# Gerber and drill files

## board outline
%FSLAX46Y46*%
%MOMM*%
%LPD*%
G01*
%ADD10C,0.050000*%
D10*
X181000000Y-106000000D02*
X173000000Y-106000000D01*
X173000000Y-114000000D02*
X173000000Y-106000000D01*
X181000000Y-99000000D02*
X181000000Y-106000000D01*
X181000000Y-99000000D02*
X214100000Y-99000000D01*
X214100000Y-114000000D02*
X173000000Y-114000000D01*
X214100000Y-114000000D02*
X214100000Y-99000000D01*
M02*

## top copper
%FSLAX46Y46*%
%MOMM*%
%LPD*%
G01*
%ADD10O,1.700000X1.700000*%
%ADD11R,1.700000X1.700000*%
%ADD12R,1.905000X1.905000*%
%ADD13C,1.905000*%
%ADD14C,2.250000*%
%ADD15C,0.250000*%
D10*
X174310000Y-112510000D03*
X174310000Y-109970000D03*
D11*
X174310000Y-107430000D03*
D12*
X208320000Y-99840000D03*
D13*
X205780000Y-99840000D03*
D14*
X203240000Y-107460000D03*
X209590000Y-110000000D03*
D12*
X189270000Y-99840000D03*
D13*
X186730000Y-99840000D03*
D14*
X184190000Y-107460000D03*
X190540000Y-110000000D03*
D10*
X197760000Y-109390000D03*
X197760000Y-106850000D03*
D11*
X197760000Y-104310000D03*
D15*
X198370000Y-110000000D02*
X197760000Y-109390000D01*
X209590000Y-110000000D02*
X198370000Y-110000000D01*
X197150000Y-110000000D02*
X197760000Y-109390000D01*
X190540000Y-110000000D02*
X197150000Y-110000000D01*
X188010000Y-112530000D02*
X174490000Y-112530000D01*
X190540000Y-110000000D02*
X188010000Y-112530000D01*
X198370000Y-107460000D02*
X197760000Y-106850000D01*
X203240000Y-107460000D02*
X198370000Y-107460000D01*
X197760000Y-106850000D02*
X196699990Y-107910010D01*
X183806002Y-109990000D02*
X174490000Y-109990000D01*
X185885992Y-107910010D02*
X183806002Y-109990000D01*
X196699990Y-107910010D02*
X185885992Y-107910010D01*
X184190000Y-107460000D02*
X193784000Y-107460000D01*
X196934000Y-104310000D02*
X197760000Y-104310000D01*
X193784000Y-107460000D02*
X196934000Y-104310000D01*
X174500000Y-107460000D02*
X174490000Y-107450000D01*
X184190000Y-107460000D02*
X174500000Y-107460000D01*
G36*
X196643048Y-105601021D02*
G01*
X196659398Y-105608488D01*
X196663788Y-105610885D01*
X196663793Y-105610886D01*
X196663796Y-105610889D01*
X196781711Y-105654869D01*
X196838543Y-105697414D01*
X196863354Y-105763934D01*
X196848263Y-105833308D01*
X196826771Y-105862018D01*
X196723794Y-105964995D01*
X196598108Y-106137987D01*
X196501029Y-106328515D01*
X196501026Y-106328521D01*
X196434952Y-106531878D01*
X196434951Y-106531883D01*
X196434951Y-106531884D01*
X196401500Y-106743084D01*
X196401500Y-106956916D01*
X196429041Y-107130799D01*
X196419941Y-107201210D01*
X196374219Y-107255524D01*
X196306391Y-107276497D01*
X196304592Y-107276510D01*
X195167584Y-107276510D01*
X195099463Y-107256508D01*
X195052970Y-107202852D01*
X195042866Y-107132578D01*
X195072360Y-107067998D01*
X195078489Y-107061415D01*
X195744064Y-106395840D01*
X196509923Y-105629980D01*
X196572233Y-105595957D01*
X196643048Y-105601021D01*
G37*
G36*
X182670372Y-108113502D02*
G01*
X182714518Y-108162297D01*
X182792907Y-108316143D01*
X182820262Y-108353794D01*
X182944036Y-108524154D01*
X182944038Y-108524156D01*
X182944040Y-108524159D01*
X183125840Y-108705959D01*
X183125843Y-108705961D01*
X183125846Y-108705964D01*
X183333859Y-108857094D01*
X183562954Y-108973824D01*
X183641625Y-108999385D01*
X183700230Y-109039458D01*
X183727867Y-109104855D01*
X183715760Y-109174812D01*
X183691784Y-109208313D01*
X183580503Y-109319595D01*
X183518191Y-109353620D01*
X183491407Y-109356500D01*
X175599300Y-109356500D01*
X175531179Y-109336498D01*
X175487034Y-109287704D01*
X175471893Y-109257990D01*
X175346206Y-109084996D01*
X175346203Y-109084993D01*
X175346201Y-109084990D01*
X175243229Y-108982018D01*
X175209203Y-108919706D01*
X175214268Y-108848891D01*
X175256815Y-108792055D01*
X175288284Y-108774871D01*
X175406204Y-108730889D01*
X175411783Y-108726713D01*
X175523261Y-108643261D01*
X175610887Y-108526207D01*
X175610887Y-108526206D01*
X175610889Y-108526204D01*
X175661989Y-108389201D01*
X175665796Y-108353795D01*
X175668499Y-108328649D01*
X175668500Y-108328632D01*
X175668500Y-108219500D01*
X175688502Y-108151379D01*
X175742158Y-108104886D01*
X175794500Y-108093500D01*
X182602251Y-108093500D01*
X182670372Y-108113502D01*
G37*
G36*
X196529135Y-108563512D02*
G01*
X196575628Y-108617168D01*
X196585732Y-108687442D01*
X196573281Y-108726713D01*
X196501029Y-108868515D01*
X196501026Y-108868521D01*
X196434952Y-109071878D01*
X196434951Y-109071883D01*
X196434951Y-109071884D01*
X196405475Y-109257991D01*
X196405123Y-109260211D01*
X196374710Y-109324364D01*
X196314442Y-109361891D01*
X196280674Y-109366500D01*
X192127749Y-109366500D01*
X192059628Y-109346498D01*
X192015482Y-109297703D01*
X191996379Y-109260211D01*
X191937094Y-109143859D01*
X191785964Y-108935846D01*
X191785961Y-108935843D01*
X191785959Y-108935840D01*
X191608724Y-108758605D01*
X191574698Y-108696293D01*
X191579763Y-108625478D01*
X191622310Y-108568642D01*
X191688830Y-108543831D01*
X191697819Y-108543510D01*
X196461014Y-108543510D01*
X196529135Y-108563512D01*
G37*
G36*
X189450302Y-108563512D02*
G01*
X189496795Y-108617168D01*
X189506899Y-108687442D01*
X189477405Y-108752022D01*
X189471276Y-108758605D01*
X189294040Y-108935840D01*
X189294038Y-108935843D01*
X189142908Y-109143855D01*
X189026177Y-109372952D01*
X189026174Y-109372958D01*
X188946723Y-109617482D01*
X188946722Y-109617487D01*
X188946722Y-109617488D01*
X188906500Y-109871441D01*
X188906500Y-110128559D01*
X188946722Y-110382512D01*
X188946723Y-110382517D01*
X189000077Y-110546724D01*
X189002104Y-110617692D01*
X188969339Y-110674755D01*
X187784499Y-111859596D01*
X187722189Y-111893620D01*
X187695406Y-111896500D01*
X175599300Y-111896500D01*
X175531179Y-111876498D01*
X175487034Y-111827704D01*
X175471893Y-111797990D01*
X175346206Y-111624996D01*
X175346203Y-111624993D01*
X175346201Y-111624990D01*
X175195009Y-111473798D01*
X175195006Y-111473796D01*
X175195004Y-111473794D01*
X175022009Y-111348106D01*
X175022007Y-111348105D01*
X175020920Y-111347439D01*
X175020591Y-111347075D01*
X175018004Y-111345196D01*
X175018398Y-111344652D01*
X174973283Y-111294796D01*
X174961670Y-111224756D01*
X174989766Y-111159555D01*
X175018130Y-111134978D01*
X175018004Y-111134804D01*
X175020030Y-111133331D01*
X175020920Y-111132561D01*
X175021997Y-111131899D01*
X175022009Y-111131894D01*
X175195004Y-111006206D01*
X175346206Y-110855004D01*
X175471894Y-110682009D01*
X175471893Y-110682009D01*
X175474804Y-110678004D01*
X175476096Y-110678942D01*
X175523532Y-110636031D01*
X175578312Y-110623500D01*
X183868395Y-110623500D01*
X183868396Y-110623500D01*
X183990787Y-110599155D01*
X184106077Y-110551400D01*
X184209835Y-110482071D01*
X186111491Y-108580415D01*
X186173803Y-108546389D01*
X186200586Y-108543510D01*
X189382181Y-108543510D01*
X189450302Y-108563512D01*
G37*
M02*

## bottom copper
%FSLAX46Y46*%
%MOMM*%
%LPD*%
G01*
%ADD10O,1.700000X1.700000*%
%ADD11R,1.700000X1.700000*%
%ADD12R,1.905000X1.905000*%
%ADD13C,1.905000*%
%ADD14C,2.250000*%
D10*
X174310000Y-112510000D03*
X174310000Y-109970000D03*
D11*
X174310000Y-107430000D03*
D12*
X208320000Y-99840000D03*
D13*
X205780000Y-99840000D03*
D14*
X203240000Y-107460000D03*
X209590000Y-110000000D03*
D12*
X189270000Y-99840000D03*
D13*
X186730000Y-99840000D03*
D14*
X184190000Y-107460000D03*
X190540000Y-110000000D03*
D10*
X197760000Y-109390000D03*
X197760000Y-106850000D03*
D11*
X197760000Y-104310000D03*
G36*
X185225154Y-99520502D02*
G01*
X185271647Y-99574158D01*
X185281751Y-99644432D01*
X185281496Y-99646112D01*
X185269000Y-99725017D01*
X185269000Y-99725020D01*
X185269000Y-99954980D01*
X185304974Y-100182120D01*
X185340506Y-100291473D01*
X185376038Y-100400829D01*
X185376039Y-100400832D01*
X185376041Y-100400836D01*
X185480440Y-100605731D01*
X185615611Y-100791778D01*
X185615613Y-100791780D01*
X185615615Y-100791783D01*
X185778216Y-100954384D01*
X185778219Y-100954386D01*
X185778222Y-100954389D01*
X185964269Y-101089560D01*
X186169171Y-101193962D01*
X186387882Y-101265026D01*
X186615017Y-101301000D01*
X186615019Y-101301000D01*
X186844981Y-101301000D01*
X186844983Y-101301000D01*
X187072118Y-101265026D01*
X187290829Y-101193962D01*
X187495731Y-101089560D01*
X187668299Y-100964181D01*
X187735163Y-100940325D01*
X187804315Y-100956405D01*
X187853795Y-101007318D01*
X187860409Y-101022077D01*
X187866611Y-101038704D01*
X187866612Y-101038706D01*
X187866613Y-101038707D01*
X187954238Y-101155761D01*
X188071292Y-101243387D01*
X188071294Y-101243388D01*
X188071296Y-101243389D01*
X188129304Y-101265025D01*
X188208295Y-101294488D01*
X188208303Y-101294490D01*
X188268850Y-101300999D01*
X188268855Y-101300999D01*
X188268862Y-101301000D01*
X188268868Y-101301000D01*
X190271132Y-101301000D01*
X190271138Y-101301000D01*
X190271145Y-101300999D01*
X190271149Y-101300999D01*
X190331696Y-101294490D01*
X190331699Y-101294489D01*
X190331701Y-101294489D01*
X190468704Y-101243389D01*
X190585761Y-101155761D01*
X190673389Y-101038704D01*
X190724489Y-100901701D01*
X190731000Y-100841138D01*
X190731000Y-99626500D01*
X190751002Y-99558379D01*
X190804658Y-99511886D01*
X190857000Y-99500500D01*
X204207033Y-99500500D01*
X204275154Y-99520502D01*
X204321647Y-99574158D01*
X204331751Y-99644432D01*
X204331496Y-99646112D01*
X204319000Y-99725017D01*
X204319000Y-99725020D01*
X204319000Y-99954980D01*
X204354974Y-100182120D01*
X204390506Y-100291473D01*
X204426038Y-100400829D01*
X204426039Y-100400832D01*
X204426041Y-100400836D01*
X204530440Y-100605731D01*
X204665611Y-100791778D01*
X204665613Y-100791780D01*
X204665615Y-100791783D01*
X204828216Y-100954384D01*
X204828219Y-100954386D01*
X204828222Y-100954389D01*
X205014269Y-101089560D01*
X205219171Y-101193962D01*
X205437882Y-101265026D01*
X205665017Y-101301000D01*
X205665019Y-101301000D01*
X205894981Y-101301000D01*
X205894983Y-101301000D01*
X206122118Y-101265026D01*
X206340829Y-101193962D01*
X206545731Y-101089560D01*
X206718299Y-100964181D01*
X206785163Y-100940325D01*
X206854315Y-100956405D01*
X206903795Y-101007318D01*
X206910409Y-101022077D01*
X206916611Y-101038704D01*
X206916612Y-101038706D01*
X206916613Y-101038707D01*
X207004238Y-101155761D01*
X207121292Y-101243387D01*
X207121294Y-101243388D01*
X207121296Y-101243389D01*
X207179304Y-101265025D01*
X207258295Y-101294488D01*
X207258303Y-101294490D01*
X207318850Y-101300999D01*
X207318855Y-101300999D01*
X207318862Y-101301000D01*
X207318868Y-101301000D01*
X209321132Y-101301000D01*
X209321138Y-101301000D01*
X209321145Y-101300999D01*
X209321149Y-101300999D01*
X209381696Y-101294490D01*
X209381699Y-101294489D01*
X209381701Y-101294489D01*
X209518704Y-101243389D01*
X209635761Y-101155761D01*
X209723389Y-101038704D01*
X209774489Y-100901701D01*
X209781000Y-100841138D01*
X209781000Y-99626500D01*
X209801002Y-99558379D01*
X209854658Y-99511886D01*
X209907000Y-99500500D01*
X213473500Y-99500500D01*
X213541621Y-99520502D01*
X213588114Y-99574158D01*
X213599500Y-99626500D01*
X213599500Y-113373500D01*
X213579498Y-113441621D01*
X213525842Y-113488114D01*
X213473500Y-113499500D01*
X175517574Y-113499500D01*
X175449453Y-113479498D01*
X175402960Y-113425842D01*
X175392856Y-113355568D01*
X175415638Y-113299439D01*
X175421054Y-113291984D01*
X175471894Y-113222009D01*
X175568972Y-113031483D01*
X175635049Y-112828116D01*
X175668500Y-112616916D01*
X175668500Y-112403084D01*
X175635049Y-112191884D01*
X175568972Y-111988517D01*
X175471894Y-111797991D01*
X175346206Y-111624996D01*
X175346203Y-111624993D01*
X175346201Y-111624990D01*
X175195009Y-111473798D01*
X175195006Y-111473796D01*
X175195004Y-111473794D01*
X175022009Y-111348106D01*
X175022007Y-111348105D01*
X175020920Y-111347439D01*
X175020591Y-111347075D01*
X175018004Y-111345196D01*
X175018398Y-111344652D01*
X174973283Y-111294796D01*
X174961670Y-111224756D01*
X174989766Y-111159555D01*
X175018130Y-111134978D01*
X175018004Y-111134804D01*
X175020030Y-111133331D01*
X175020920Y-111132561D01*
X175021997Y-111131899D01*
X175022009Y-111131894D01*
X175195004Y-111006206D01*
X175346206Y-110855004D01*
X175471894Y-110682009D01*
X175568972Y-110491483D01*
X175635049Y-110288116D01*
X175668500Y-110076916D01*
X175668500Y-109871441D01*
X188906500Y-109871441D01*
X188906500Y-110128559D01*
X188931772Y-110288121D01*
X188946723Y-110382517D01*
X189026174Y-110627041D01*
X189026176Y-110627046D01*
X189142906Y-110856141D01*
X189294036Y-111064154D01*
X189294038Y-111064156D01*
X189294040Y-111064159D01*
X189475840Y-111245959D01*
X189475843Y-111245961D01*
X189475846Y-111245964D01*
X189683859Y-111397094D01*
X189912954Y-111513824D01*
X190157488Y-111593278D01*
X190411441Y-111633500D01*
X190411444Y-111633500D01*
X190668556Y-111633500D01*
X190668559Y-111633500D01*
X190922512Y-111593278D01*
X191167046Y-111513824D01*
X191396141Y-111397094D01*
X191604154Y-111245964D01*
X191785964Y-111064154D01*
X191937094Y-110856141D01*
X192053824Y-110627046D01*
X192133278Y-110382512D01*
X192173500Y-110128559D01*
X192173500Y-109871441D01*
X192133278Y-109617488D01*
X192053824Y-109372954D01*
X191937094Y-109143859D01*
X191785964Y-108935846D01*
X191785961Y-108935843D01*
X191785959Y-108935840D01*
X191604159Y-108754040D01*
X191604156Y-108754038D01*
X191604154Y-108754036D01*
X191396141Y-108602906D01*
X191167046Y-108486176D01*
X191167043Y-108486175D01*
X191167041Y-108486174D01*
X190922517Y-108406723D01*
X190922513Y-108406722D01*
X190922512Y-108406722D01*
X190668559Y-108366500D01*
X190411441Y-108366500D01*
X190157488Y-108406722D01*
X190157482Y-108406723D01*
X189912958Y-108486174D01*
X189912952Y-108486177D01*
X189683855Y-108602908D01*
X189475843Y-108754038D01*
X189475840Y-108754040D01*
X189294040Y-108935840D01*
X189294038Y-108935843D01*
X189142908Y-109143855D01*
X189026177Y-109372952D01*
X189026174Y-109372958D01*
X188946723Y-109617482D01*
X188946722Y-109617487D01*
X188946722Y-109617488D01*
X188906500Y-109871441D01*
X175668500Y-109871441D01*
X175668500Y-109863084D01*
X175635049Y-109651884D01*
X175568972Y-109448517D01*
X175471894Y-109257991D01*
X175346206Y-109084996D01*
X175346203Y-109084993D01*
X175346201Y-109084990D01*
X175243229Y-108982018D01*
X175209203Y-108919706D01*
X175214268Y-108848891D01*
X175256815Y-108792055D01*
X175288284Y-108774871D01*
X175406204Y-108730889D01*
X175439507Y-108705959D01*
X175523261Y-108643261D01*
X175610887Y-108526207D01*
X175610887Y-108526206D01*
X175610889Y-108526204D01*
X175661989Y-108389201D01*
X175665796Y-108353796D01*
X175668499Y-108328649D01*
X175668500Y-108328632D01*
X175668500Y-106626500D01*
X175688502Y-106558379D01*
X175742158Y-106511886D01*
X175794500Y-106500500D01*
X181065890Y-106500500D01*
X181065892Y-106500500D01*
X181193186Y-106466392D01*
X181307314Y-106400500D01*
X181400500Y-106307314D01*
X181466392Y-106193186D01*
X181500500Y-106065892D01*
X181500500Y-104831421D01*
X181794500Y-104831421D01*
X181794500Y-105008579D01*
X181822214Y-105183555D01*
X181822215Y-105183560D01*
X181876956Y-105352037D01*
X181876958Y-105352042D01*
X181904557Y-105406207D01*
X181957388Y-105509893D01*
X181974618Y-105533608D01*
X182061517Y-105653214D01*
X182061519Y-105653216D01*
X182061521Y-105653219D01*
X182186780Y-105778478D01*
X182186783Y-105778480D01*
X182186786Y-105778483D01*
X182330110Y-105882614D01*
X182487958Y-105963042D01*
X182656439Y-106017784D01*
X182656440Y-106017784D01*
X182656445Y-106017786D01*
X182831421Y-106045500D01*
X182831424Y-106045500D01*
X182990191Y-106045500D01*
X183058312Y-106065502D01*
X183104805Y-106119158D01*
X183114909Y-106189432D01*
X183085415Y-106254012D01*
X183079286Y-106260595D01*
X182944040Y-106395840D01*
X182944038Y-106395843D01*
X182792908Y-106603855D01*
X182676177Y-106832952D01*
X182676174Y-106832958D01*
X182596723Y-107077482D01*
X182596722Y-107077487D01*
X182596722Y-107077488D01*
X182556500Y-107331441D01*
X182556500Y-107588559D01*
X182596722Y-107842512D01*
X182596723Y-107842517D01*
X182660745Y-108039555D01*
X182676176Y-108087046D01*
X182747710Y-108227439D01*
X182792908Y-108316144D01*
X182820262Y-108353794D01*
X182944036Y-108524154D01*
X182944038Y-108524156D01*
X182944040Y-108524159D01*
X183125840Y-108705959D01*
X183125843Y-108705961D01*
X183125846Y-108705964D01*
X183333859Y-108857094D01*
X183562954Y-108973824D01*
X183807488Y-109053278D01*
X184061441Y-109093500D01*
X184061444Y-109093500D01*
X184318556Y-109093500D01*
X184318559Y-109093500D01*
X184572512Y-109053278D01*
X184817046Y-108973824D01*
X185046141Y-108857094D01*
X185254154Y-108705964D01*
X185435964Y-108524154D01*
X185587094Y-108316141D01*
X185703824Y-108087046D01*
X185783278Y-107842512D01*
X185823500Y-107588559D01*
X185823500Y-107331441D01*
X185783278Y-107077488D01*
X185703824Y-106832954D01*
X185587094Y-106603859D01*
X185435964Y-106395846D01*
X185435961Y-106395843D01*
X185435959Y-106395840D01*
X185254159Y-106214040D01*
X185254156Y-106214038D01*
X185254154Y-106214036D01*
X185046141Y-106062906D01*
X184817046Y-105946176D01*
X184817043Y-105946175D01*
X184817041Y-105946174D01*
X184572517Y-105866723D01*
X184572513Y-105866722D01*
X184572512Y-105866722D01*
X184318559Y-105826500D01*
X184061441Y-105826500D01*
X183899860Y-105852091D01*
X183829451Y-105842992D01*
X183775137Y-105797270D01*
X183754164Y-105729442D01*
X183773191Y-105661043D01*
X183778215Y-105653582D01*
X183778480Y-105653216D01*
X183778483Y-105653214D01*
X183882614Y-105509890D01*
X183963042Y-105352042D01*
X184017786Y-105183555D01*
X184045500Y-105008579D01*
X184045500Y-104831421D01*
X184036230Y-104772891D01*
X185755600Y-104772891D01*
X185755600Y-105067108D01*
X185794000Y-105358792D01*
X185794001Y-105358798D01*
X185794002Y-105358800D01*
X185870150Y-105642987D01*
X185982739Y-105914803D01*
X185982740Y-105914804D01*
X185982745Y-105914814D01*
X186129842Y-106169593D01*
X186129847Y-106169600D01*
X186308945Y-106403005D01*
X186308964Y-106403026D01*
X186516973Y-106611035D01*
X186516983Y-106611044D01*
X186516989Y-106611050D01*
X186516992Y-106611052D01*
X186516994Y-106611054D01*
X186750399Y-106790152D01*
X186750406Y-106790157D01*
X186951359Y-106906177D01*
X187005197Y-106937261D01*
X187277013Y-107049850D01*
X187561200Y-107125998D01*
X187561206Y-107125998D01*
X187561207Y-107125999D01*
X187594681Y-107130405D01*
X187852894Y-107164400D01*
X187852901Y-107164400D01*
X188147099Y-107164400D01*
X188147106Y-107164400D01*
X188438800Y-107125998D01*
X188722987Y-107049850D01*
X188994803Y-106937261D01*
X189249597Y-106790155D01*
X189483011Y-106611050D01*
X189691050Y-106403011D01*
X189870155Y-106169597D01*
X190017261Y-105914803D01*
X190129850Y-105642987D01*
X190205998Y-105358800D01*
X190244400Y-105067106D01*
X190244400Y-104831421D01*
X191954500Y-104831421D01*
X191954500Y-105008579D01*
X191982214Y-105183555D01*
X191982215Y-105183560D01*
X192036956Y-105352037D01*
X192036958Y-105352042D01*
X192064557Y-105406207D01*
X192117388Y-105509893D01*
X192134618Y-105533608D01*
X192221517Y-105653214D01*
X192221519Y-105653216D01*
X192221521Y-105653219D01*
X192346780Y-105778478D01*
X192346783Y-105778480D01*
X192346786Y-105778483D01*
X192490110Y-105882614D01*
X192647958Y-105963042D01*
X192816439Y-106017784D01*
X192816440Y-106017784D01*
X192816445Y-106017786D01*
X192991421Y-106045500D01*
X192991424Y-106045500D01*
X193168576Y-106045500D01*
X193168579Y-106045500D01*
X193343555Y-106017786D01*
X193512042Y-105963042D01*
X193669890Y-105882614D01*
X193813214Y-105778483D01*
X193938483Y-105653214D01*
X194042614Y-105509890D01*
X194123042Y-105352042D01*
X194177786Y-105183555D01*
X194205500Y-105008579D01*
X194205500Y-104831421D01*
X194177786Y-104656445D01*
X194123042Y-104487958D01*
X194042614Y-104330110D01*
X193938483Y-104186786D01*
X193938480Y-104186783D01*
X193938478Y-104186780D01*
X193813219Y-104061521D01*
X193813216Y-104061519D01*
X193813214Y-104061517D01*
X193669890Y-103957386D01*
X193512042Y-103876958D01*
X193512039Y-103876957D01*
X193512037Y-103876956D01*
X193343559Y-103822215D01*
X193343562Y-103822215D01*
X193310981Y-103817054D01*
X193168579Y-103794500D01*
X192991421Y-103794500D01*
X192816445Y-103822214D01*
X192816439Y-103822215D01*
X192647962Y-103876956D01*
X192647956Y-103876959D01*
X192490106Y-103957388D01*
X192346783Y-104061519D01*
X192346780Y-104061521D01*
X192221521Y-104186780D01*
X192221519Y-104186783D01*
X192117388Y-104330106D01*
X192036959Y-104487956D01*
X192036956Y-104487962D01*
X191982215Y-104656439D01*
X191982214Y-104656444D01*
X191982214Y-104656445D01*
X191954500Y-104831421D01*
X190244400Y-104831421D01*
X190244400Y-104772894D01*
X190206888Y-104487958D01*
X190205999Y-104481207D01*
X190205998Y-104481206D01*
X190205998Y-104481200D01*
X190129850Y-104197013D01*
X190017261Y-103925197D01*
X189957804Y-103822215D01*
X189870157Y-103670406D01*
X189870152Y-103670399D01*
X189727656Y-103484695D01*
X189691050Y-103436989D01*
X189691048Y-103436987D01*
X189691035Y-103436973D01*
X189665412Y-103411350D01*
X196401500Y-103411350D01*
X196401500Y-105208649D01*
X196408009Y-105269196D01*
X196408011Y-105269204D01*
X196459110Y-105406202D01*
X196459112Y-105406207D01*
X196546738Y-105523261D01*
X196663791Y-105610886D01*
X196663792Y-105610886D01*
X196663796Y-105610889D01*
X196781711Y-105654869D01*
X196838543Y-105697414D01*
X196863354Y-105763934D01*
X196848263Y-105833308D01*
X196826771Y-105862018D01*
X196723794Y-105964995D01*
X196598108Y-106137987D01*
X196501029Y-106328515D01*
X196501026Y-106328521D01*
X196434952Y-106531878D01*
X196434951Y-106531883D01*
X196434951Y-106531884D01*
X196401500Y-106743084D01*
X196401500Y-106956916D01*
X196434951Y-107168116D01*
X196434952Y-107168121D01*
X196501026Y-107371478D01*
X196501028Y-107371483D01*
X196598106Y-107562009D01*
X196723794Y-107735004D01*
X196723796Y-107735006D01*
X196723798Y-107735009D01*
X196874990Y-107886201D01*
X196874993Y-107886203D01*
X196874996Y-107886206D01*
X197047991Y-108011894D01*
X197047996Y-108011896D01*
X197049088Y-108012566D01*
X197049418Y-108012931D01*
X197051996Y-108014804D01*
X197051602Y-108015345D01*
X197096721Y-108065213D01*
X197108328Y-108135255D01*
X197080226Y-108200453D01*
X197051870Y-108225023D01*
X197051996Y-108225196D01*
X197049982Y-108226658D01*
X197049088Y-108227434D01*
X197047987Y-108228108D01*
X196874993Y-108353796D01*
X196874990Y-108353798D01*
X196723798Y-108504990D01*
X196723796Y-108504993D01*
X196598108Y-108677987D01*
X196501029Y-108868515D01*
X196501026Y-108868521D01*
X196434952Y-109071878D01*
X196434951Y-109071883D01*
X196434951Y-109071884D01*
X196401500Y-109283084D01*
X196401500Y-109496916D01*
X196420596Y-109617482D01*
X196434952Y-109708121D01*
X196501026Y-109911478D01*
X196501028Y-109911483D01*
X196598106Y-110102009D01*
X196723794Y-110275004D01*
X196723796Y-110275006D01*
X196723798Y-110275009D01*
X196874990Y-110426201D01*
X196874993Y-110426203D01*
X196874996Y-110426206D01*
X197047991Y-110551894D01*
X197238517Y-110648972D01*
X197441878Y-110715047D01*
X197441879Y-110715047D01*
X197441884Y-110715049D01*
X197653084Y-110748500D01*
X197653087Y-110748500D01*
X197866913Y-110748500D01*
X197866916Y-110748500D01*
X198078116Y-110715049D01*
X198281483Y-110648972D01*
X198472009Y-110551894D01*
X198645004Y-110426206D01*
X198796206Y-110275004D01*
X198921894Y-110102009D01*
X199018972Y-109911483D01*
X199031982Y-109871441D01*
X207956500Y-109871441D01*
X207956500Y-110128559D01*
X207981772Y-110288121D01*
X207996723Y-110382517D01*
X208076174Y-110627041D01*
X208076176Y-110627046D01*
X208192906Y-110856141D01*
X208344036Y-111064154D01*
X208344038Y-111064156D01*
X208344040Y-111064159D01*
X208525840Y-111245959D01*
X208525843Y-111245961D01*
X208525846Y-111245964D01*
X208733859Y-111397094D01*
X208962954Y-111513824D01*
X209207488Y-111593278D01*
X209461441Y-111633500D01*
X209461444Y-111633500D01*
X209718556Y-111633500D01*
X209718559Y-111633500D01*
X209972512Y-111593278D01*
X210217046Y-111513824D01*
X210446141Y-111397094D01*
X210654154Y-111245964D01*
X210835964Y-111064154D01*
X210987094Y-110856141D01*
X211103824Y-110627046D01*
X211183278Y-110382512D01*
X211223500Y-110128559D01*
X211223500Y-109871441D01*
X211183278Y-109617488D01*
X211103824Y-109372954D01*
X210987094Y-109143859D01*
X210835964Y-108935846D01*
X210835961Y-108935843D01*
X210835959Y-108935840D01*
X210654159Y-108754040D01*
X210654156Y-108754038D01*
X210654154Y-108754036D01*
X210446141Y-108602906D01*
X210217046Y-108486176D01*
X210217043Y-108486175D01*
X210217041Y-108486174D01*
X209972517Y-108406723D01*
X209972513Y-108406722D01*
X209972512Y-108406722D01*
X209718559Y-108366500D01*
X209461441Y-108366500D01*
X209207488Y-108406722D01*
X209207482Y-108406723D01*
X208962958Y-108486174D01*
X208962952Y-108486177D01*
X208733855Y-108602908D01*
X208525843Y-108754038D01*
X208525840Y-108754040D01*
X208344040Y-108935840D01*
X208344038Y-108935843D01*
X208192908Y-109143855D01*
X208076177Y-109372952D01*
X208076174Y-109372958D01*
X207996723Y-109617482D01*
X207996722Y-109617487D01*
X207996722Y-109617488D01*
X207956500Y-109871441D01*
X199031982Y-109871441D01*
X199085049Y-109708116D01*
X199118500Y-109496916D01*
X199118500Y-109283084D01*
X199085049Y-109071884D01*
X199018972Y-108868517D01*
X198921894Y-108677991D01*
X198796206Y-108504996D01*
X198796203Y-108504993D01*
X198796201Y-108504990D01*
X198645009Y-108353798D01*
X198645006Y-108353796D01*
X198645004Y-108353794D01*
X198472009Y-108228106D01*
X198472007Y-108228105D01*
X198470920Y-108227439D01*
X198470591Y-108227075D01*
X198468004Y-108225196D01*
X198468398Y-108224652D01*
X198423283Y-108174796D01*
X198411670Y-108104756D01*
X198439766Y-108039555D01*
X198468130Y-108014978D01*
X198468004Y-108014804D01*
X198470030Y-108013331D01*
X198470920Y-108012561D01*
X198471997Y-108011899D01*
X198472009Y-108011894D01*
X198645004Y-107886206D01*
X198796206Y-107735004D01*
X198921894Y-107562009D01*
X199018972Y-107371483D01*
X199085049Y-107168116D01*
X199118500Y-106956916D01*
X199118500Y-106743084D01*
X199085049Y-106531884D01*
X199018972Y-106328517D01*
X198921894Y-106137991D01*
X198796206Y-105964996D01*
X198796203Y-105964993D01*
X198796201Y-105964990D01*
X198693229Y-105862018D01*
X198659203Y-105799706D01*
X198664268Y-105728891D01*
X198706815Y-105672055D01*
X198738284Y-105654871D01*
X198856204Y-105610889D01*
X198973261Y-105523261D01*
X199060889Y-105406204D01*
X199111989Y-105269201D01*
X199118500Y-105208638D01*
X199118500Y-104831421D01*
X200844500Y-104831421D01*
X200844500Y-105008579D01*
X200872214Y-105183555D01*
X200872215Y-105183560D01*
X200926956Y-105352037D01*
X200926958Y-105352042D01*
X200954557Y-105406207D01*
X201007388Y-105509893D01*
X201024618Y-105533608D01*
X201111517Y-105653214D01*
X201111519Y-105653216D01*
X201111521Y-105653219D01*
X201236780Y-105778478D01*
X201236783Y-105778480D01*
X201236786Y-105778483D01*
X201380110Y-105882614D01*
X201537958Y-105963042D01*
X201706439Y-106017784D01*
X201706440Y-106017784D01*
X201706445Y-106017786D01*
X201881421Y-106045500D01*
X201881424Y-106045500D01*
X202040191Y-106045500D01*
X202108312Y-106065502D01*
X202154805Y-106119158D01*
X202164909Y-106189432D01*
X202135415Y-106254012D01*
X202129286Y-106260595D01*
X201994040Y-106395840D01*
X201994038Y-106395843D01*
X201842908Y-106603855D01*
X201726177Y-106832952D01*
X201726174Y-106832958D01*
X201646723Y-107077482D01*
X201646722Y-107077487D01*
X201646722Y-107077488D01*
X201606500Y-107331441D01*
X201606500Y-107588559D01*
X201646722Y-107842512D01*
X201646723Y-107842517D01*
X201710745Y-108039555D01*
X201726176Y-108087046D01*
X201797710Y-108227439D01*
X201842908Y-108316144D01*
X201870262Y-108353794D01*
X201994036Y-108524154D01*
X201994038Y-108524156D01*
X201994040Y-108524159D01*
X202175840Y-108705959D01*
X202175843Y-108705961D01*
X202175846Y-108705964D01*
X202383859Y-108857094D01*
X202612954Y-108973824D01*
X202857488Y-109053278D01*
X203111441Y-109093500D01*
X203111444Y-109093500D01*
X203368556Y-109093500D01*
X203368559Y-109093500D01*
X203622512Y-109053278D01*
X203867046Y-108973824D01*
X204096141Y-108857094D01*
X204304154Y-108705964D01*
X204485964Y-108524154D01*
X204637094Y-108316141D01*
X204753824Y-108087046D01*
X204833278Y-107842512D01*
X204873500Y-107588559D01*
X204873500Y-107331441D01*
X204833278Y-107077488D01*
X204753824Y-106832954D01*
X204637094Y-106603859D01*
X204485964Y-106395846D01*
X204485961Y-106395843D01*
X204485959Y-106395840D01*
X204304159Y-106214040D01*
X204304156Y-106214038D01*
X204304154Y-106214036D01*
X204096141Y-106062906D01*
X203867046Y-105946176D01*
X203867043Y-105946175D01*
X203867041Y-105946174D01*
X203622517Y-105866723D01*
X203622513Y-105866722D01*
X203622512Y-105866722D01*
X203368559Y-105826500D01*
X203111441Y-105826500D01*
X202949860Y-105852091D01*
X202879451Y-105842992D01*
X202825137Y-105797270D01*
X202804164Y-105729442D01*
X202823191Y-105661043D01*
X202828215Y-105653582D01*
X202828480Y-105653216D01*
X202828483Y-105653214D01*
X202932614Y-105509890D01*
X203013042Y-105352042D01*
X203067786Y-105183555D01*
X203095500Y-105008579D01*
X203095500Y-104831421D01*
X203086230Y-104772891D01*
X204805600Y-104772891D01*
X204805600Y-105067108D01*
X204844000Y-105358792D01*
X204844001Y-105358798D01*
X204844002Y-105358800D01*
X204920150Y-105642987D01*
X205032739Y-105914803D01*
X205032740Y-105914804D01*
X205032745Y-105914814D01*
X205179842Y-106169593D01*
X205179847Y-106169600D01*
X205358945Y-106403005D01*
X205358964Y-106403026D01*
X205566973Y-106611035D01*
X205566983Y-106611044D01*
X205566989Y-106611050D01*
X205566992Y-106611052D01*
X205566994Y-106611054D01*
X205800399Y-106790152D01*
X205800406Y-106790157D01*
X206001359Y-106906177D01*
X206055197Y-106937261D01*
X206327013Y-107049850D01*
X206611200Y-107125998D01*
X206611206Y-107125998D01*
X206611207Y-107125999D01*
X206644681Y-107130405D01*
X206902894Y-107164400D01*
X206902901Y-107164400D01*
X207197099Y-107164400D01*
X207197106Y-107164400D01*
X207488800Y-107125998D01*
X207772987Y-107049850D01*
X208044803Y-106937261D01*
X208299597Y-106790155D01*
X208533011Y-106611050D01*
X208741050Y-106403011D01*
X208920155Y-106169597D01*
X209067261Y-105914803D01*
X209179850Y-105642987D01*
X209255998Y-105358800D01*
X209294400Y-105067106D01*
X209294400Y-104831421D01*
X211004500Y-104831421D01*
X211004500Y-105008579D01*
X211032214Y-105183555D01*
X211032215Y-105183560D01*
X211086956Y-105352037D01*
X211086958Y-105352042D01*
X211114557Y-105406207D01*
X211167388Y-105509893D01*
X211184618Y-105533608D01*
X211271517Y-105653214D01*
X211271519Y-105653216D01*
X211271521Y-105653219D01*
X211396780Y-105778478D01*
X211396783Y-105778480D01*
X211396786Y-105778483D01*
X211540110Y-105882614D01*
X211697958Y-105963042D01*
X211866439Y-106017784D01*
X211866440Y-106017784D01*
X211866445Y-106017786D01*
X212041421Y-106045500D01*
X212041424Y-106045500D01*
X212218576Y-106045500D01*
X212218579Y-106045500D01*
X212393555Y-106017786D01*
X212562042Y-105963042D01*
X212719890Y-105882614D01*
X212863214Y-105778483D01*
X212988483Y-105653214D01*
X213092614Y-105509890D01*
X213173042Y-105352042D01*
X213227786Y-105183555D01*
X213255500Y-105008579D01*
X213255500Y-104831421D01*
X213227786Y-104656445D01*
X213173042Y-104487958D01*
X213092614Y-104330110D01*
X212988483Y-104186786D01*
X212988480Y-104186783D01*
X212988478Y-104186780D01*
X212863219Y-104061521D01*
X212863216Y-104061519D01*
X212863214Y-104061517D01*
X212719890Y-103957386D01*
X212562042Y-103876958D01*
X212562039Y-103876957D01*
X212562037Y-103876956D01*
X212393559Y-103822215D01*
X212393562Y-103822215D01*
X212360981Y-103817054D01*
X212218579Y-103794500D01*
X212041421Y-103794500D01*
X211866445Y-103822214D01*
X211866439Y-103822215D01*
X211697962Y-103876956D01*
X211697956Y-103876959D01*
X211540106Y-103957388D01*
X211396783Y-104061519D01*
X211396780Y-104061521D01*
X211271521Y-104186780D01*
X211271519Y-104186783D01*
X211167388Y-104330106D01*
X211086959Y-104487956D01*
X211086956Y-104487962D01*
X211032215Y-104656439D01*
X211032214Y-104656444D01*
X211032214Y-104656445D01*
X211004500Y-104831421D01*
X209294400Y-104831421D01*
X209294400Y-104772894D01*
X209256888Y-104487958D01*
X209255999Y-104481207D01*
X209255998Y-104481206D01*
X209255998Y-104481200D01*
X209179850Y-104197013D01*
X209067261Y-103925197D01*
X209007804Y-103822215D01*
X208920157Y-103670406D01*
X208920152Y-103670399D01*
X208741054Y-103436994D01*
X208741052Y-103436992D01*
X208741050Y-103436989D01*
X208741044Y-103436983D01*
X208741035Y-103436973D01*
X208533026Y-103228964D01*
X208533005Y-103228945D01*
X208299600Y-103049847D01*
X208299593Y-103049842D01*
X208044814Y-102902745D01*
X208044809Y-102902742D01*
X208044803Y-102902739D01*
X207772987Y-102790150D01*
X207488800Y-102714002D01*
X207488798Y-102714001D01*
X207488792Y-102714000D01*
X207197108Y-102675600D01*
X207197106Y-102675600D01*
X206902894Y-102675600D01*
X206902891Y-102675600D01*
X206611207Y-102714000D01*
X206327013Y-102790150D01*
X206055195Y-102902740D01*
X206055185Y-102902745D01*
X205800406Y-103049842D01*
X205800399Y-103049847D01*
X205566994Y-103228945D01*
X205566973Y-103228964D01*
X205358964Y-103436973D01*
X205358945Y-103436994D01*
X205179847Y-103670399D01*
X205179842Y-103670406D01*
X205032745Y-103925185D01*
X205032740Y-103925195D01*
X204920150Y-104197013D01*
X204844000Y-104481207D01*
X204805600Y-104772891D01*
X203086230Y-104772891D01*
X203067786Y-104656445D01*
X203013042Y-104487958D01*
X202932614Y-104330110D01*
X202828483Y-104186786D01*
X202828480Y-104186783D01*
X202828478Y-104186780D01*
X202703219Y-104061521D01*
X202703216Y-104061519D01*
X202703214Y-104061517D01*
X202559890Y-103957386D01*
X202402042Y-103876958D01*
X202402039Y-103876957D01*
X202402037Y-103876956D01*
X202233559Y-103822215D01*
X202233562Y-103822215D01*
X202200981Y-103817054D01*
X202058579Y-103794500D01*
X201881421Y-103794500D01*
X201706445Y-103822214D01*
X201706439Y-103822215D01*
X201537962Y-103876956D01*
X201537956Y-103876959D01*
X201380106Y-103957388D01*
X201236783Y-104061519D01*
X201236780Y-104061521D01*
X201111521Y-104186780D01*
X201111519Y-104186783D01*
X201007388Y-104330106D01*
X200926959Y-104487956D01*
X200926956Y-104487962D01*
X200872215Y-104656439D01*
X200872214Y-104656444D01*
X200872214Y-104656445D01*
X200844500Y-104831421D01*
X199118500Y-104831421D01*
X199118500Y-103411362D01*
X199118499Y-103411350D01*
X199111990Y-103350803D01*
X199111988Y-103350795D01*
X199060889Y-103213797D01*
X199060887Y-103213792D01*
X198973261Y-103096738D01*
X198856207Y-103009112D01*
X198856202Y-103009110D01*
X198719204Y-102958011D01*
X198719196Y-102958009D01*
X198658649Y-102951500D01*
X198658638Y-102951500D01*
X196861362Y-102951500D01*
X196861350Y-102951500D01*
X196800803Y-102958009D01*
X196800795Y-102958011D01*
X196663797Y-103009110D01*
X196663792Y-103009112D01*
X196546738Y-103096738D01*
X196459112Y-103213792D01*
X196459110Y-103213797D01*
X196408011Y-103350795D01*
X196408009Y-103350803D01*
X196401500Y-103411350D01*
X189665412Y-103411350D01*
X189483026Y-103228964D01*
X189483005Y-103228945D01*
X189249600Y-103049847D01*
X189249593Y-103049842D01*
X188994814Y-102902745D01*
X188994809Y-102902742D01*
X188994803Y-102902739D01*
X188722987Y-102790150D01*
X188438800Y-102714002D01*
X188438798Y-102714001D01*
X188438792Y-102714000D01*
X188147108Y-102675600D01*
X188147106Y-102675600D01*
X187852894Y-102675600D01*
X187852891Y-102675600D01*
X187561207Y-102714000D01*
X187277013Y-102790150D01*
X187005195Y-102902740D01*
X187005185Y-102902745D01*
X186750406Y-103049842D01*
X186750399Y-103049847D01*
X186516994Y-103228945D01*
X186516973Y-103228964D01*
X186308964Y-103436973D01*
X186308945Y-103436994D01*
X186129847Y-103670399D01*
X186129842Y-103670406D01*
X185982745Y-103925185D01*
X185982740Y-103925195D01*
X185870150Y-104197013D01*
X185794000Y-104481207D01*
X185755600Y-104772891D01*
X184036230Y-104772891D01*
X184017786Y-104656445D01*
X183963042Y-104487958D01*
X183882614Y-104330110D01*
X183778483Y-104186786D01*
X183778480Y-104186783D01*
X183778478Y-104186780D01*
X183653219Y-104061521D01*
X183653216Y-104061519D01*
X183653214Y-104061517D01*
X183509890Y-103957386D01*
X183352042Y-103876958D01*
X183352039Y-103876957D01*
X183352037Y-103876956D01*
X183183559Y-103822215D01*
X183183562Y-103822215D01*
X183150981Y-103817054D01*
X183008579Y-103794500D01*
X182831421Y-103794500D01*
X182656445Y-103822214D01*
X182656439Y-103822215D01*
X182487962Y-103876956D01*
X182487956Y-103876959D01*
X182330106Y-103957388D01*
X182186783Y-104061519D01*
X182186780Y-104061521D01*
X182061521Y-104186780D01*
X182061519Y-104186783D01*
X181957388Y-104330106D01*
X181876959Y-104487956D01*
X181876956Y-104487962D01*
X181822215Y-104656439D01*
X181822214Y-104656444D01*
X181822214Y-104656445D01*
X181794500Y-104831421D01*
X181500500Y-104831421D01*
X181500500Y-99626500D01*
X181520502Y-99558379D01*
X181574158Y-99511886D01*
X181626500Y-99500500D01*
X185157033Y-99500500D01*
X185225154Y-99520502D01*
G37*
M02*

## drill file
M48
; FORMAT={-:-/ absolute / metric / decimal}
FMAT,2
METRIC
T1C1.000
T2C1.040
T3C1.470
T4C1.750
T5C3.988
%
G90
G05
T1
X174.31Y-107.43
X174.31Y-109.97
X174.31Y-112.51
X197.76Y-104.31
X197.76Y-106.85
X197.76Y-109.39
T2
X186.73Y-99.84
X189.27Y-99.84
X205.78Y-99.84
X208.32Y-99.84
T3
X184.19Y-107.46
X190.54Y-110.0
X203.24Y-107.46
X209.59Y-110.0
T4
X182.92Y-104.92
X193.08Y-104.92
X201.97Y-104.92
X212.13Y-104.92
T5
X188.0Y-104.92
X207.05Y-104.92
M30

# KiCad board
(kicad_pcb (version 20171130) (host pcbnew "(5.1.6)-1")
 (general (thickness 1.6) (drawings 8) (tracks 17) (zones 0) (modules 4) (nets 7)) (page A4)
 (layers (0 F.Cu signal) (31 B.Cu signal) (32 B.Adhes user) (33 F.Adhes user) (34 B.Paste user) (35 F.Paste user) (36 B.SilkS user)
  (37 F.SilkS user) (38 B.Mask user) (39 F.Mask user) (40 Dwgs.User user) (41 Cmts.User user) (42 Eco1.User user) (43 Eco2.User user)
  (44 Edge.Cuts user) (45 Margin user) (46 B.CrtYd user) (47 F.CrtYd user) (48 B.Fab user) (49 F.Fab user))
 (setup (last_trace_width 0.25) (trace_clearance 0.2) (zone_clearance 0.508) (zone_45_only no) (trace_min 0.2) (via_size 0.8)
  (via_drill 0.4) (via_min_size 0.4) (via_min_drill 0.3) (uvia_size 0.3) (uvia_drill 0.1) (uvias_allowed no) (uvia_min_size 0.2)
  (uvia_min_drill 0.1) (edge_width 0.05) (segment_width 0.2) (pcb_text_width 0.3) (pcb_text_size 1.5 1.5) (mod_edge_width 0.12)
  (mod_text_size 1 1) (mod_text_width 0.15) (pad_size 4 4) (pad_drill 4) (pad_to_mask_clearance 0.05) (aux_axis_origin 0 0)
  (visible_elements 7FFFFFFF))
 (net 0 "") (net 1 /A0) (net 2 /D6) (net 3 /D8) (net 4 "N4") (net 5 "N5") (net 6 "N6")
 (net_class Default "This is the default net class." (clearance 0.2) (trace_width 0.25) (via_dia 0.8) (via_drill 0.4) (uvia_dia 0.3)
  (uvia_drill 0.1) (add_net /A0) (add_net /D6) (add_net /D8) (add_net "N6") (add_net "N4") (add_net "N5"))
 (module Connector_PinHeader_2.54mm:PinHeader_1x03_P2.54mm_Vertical (layer F.Cu) (at 174.31 107.43)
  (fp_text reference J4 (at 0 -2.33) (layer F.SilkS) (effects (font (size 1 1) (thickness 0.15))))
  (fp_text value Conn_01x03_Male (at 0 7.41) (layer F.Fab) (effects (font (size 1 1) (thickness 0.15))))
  (pad 3 thru_hole oval (at 0 5.08) (size 1.7 1.7) (drill 1) (layers *.Cu *.Mask) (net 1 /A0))
  (pad 2 thru_hole oval (at 0 2.54) (size 1.7 1.7) (drill 1) (layers *.Cu *.Mask) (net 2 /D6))
  (pad 1 thru_hole rect (at 0 0) (size 1.7 1.7) (drill 1) (layers *.Cu *.Mask) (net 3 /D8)))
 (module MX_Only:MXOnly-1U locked (layer B.Cu) (at 207.05 104.92)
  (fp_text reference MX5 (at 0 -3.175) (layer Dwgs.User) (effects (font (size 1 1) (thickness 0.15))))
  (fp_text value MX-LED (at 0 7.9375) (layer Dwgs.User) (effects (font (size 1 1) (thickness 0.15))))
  (pad "" np_thru_hole circle (at 5.08 0 311.9004) (size 1.75 1.75) (drill 1.75) (layers *.Cu *.Mask))
  (pad "" np_thru_hole circle (at -5.08 0 311.9004) (size 1.75 1.75) (drill 1.75) (layers *.Cu *.Mask))
  (pad 4 thru_hole rect (at 1.27 -5.08) (size 1.905 1.905) (drill 1.04) (layers *.Cu F.Mask) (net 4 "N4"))
  (pad 3 thru_hole circle (at -1.27 -5.08) (size 1.905 1.905) (drill 1.04) (layers *.Cu F.Mask) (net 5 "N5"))
  (pad 1 thru_hole circle (at -3.81 2.54) (size 2.25 2.25) (drill 1.47) (layers *.Cu F.Mask) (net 2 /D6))
  (pad "" np_thru_hole circle (at 0 0) (size 3.9878 3.9878) (drill 3.9878) (layers *.Cu *.Mask))
  (pad 2 thru_hole circle (at 2.54 5.08) (size 2.25 2.25) (drill 1.47) (layers *.Cu F.Mask) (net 1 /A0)))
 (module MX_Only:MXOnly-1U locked (layer B.Cu) (at 188 104.92)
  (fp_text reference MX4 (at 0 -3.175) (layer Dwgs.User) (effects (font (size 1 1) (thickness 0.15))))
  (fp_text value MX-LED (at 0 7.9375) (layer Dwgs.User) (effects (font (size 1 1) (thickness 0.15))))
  (pad "" np_thru_hole circle (at 5.08 0 311.9004) (size 1.75 1.75) (drill 1.75) (layers *.Cu *.Mask))
  (pad "" np_thru_hole circle (at -5.08 0 311.9004) (size 1.75 1.75) (drill 1.75) (layers *.Cu *.Mask))
  (pad 4 thru_hole rect (at 1.27 -5.08) (size 1.905 1.905) (drill 1.04) (layers *.Cu F.Mask) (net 4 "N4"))
  (pad 3 thru_hole circle (at -1.27 -5.08) (size 1.905 1.905) (drill 1.04) (layers *.Cu F.Mask) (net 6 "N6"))
  (pad 1 thru_hole circle (at -3.81 2.54) (size 2.25 2.25) (drill 1.47) (layers *.Cu F.Mask) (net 3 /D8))
  (pad "" np_thru_hole circle (at 0 0) (size 3.9878 3.9878) (drill 3.9878) (layers *.Cu *.Mask))
  (pad 2 thru_hole circle (at 2.54 5.08) (size 2.25 2.25) (drill 1.47) (layers *.Cu F.Mask) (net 1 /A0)))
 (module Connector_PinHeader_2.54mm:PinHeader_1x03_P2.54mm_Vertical (layer F.Cu) (at 197.76 104.31)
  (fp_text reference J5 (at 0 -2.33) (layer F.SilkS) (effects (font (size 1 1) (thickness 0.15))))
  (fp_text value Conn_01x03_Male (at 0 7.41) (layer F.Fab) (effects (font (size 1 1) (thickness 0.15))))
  (pad 3 thru_hole oval (at 0 5.08) (size 1.7 1.7) (drill 1) (layers *.Cu *.Mask) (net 1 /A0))
  (pad 2 thru_hole oval (at 0 2.54) (size 1.7 1.7) (drill 1) (layers *.Cu *.Mask) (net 2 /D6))
  (pad 1 thru_hole rect (at 0 0) (size 1.7 1.7) (drill 1) (layers *.Cu *.Mask) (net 3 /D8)))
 (gr_line (start 181 106) (end 173 106) (layer Edge.Cuts) (width 0.05))
 (gr_line (start 173 114) (end 173 106) (layer Edge.Cuts) (width 0.05))
 (gr_line (start 181 99) (end 181 106) (layer Edge.Cuts) (width 0.05))
 (gr_line (start 181 99) (end 214.1 99) (layer Edge.Cuts) (width 0.05))
 (gr_line (start 214.1 114) (end 173 114) (layer Edge.Cuts) (width 0.05))
 (gr_line (start 214.1 114) (end 214.1 99) (layer Edge.Cuts) (width 0.05))
 (segment (start 198.37 110) (end 197.76 109.39) (width 0.25) (layer F.Cu) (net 1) (status 20))
 (segment (start 209.59 110) (end 198.37 110) (width 0.25) (layer F.Cu) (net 1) (status 10))
 (segment (start 197.15 110) (end 197.76 109.39) (width 0.25) (layer F.Cu) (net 1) (status 20))
 (segment (start 190.54 110) (end 197.15 110) (width 0.25) (layer F.Cu) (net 1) (status 10))
 (segment (start 188.01 112.53) (end 174.49 112.53) (width 0.25) (layer F.Cu) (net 1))
 (segment (start 190.54 110) (end 188.01 112.53) (width 0.25) (layer F.Cu) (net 1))
 (segment (start 198.37 107.46) (end 197.76 106.85) (width 0.25) (layer F.Cu) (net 2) (status 20))
 (segment (start 203.24 107.46) (end 198.37 107.46) (width 0.25) (layer F.Cu) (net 2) (status 10))
 (segment (start 197.76 106.85) (end 196.69999 107.91001) (width 0.25) (layer F.Cu) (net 2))
 (segment (start 183.806002 109.99) (end 174.49 109.99) (width 0.25) (layer F.Cu) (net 2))
 (segment (start 185.885992 107.91001) (end 183.806002 109.99) (width 0.25) (layer F.Cu) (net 2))
 (segment (start 196.69999 107.91001) (end 185.885992 107.91001) (width 0.25) (layer F.Cu) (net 2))
 (segment (start 184.19 107.46) (end 193.784 107.46) (width 0.25) (layer F.Cu) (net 3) (status 10))
 (segment (start 196.934 104.31) (end 197.76 104.31) (width 0.25) (layer F.Cu) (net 3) (status 30))
 (segment (start 193.784 107.46) (end 196.934 104.31) (width 0.25) (layer F.Cu) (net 3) (status 20))
 (segment (start 174.5 107.46) (end 174.49 107.45) (width 0.25) (layer F.Cu) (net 3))
 (segment (start 184.19 107.46) (end 174.5 107.46) (width 0.25) (layer F.Cu) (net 3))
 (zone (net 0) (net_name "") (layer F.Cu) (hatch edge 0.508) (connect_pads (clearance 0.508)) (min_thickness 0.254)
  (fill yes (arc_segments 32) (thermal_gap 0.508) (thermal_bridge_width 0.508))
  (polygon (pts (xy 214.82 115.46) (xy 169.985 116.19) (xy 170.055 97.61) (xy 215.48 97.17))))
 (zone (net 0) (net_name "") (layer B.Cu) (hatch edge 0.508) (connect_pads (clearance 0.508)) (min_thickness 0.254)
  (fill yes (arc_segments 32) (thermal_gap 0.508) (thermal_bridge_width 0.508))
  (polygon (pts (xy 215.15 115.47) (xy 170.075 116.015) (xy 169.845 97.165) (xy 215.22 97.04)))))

